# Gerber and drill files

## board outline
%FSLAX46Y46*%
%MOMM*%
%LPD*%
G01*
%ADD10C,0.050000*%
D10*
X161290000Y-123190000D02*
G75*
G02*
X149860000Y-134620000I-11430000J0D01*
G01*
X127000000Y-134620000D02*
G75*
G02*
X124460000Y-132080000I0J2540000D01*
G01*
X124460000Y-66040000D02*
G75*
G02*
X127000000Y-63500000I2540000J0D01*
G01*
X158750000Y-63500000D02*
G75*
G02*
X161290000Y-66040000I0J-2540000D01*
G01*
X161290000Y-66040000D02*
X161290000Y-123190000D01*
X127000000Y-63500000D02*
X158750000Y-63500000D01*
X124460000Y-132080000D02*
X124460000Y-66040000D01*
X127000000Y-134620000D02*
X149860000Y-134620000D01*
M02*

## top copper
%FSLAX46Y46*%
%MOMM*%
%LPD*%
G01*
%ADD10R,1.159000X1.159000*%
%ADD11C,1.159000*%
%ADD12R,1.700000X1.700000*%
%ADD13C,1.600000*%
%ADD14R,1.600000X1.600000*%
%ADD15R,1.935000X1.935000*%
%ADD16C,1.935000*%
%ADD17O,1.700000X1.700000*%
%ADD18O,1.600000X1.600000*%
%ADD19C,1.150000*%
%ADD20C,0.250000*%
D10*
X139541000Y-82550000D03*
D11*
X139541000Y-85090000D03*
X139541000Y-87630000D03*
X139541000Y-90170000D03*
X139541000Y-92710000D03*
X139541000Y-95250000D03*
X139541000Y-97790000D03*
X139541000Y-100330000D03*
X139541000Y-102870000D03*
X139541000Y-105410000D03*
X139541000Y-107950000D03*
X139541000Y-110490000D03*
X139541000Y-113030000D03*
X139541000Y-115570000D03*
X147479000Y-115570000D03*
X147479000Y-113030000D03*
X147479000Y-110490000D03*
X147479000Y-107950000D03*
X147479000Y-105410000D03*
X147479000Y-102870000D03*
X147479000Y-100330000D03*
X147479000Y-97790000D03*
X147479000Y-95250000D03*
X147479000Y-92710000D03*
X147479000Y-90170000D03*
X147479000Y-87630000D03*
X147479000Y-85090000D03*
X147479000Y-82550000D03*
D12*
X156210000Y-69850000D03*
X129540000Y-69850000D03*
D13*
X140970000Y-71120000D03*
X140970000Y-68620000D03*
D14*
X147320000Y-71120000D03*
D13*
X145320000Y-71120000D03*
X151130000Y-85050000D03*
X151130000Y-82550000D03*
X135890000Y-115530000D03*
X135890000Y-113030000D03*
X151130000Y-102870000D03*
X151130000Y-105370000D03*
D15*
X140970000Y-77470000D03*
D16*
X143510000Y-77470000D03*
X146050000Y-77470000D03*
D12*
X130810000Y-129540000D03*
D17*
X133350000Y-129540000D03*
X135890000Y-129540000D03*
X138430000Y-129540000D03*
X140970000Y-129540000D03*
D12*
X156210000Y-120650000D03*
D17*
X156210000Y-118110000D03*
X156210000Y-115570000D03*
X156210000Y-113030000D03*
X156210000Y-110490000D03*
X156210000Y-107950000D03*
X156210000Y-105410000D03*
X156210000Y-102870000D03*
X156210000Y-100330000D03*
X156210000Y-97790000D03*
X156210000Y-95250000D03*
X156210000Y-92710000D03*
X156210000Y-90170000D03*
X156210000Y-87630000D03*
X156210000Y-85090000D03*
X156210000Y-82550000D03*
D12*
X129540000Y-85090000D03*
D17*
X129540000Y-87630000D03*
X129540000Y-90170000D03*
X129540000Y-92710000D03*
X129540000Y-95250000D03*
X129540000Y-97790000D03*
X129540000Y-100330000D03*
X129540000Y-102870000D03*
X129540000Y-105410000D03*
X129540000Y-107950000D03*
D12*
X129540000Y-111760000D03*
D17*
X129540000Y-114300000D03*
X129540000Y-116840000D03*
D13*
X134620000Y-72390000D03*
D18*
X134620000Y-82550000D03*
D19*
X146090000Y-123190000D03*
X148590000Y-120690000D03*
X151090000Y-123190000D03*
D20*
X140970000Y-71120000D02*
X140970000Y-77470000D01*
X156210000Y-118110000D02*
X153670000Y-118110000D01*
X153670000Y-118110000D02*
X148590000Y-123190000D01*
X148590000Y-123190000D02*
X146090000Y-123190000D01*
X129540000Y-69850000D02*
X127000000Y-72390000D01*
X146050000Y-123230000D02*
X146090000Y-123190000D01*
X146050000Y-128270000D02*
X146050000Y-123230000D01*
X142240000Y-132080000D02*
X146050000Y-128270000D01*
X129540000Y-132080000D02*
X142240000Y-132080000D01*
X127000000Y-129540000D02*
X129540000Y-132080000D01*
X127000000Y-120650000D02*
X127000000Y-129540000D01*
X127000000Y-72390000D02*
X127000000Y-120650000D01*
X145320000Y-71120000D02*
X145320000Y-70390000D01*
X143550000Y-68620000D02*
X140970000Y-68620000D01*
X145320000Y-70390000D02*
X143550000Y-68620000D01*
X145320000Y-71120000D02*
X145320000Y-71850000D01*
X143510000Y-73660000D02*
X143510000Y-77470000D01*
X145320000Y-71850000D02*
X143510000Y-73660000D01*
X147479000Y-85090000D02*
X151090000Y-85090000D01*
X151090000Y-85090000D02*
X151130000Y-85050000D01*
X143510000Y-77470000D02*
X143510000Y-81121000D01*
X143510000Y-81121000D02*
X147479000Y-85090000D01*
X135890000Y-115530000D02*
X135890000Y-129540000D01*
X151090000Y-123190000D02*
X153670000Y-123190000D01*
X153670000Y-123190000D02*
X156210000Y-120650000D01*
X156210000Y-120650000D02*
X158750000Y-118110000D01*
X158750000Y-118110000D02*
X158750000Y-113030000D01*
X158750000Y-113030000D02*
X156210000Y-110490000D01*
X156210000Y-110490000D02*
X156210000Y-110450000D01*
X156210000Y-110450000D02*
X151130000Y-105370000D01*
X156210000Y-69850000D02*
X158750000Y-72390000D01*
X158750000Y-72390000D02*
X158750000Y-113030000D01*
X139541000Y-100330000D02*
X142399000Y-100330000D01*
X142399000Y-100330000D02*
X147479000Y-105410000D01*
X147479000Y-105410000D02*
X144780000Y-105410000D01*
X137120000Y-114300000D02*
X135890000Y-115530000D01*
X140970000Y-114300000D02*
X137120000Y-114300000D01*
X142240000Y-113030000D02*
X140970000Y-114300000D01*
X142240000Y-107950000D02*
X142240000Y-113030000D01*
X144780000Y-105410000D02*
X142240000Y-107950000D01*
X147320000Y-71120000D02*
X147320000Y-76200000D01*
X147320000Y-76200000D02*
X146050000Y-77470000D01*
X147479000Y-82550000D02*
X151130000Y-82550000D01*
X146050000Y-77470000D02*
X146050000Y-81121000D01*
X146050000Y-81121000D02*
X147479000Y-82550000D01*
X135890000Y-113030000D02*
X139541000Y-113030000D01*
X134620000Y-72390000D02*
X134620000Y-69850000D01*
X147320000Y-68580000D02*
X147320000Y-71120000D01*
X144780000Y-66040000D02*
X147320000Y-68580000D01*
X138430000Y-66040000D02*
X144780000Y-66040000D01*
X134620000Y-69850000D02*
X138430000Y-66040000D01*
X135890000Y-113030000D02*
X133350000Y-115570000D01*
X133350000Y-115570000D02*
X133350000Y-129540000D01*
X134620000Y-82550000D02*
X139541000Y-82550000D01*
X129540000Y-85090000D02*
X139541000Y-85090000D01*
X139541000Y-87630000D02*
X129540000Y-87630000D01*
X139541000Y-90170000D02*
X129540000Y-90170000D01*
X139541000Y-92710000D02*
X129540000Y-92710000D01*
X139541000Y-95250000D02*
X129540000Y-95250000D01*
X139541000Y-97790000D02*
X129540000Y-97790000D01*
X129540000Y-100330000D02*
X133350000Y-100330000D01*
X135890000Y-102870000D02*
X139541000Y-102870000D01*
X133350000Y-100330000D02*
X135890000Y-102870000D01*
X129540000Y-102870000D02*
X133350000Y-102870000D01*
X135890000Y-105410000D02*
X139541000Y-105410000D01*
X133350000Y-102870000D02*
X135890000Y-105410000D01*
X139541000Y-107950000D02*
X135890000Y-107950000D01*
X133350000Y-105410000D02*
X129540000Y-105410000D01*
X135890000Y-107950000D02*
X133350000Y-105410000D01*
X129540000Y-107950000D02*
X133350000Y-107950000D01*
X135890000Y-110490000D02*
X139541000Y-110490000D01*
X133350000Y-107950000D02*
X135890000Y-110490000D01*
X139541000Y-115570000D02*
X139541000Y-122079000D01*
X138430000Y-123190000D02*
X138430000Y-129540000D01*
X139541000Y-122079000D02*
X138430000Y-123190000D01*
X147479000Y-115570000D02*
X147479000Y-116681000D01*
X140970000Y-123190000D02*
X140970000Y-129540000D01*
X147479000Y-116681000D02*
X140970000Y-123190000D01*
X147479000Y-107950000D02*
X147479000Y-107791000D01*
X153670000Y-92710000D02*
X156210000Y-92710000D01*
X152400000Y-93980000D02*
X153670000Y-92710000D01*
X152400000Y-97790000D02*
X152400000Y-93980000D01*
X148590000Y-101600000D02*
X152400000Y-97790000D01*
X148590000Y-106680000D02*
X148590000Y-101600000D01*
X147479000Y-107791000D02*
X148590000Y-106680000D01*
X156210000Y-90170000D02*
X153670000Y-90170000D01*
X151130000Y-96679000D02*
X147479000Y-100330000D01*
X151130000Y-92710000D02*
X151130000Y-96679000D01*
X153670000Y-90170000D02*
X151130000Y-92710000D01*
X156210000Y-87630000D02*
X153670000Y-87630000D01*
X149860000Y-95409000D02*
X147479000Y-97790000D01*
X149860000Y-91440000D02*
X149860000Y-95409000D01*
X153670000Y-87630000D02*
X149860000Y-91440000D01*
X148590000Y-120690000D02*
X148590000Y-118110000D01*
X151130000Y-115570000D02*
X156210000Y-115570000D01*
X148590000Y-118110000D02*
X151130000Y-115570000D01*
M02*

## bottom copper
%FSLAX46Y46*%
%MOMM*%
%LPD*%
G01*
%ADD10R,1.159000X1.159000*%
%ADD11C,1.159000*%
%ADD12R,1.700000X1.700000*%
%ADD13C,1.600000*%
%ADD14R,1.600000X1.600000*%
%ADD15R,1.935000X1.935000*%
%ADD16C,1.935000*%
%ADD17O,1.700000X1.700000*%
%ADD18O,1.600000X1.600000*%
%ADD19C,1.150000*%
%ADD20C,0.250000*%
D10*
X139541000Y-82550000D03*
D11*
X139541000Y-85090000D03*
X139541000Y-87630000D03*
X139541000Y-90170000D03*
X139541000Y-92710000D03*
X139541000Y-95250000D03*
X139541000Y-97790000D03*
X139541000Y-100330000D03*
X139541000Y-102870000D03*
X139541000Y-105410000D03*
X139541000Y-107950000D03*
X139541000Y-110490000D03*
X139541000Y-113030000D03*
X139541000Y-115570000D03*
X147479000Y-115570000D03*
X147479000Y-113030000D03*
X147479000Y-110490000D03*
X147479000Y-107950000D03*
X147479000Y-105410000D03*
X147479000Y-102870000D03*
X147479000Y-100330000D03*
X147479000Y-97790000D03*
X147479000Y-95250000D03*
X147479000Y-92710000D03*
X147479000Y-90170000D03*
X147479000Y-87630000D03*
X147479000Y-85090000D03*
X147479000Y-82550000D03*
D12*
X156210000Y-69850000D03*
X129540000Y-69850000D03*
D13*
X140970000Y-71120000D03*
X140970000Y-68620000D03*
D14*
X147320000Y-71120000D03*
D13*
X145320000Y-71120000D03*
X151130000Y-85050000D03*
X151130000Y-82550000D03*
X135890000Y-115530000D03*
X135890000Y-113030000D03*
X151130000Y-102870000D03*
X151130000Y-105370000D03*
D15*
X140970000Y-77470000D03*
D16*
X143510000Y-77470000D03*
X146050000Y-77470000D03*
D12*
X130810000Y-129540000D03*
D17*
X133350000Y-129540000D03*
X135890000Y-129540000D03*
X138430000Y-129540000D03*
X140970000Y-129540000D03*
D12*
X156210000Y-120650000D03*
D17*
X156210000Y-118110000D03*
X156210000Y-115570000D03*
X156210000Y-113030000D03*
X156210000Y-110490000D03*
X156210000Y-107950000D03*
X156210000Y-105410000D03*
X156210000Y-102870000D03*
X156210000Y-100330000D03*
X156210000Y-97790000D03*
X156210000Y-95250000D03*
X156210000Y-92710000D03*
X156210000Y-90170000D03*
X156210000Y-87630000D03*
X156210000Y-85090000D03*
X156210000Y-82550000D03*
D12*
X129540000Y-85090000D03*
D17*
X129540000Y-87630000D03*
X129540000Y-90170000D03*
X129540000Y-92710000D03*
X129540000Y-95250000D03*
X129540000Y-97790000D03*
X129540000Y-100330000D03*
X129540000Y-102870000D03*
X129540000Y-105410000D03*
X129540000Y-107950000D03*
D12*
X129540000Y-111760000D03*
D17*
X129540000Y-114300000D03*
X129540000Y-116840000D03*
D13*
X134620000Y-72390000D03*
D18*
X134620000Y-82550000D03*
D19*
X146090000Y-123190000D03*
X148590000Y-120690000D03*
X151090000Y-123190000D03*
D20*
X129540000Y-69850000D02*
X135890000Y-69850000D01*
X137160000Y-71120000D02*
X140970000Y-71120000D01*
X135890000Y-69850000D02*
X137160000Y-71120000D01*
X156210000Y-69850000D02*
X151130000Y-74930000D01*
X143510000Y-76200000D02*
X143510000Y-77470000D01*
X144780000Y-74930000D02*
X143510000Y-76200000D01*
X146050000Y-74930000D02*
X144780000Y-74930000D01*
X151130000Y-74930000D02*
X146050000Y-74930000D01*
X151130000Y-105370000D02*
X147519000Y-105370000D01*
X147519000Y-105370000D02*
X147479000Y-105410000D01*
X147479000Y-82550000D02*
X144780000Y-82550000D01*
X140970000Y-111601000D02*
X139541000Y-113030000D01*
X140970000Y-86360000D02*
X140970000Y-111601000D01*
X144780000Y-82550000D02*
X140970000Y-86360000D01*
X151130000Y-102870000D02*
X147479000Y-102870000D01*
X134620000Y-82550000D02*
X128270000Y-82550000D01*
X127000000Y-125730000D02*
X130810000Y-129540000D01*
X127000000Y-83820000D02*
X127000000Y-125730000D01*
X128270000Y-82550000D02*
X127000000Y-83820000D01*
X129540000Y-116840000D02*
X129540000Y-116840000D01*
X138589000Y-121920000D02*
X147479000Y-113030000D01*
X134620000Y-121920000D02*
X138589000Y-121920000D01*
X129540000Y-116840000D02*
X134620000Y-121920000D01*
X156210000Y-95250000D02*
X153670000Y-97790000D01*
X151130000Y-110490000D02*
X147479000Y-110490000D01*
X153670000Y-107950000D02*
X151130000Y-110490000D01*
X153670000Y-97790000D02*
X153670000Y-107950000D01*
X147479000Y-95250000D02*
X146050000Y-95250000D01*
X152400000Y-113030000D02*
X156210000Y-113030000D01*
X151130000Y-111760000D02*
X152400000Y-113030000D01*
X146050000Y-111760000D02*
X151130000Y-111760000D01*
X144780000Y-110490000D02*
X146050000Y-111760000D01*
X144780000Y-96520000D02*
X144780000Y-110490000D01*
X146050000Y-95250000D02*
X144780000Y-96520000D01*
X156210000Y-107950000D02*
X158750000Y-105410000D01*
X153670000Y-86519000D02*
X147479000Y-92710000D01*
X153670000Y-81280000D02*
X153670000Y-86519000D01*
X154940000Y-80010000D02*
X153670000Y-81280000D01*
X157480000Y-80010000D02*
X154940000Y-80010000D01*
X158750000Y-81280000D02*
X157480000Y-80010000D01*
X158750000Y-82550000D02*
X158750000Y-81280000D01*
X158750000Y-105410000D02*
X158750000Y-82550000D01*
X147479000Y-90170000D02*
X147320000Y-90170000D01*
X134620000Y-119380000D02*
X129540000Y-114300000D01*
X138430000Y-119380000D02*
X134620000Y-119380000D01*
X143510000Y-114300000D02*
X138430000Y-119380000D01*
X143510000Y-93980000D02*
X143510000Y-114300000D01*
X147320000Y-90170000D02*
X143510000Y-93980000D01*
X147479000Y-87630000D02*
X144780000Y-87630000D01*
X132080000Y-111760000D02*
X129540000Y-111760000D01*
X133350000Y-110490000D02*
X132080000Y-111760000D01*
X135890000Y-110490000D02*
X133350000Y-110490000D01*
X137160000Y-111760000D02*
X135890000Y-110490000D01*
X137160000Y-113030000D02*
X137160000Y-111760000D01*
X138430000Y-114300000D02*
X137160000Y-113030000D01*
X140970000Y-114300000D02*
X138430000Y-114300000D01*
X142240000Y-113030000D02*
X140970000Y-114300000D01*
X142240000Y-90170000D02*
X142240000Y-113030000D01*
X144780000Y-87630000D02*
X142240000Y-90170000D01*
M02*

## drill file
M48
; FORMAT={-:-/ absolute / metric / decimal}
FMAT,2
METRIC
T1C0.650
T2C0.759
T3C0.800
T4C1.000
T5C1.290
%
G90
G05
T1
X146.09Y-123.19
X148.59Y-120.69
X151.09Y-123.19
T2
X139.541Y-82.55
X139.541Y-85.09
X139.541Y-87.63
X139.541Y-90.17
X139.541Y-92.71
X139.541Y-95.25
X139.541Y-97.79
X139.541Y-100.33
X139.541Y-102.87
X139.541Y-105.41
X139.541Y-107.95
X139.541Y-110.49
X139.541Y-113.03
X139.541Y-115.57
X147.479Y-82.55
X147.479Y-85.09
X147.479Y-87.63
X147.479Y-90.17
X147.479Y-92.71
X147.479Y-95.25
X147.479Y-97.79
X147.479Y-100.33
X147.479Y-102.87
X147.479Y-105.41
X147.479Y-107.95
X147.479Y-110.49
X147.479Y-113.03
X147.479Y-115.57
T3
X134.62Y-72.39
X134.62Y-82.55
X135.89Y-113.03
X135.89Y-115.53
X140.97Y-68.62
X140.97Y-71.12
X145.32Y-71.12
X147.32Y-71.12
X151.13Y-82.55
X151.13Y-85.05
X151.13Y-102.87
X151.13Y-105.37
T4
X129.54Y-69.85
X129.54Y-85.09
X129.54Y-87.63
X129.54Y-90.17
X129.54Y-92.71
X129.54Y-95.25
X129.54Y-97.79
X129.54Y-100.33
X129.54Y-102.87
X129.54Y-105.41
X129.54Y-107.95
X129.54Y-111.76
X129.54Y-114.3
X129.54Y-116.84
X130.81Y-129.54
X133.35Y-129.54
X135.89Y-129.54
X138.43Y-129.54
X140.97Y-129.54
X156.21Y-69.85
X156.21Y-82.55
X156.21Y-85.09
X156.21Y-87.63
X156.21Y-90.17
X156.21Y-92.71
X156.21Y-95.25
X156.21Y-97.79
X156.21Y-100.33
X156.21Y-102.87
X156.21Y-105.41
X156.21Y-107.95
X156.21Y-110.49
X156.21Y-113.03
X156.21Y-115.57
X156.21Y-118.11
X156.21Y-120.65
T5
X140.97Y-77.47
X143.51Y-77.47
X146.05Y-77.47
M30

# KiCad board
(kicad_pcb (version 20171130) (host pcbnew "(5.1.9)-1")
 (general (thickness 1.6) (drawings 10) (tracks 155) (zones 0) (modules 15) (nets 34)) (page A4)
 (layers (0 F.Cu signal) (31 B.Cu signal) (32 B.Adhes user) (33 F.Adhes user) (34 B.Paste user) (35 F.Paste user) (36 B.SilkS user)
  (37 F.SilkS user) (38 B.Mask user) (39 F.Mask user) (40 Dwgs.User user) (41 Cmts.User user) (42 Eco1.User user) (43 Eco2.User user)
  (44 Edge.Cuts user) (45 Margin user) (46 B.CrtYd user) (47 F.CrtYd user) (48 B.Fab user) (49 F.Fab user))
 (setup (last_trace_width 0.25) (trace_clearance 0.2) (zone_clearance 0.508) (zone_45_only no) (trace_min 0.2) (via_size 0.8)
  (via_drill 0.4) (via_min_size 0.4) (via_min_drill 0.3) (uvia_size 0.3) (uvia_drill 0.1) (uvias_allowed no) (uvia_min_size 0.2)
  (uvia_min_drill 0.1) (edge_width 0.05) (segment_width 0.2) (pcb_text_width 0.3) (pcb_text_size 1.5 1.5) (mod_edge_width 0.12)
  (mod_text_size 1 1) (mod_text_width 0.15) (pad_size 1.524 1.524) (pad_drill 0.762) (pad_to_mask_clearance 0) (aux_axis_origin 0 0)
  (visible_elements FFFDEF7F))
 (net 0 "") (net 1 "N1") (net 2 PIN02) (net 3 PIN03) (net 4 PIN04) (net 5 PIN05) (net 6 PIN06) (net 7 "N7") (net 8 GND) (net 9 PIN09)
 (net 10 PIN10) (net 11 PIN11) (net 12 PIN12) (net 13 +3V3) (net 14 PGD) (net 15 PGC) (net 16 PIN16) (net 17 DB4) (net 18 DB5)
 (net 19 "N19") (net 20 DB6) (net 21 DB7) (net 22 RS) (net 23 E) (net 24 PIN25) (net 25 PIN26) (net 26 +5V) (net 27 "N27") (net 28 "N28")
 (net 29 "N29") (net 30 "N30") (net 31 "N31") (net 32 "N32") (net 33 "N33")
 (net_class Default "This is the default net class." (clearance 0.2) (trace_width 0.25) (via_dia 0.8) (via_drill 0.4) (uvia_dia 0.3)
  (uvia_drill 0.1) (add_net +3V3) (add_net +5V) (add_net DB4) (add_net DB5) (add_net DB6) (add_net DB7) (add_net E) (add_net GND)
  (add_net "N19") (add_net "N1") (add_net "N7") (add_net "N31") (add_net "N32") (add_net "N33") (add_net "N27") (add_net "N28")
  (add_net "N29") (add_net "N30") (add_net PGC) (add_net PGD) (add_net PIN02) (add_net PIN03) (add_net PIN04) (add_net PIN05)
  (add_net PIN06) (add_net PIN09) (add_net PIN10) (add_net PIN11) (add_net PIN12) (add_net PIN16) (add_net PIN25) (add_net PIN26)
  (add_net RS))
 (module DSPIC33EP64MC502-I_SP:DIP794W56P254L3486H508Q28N (layer F.Cu) (at 143.51 99.06)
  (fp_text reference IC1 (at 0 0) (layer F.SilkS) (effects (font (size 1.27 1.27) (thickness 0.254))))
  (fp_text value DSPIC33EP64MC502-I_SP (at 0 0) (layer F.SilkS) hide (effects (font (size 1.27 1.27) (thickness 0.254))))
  (pad 1 thru_hole rect (at -3.969 -16.51 90) (size 1.159 1.159) (drill 0.759) (layers *.Cu *.Mask F.SilkS) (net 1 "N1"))
  (pad 2 thru_hole circle (at -3.969 -13.97 90) (size 1.159 1.159) (drill 0.759) (layers *.Cu *.Mask F.SilkS) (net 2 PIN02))
  (pad 3 thru_hole circle (at -3.969 -11.43 90) (size 1.159 1.159) (drill 0.759) (layers *.Cu *.Mask F.SilkS) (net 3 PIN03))
  (pad 4 thru_hole circle (at -3.969 -8.89 90) (size 1.159 1.159) (drill 0.759) (layers *.Cu *.Mask F.SilkS) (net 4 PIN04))
  (pad 5 thru_hole circle (at -3.969 -6.35 90) (size 1.159 1.159) (drill 0.759) (layers *.Cu *.Mask F.SilkS) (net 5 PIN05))
  (pad 6 thru_hole circle (at -3.969 -3.81 90) (size 1.159 1.159) (drill 0.759) (layers *.Cu *.Mask F.SilkS) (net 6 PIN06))
  (pad 7 thru_hole circle (at -3.969 -1.27 90) (size 1.159 1.159) (drill 0.759) (layers *.Cu *.Mask F.SilkS) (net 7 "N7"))
  (pad 8 thru_hole circle (at -3.969 1.27 90) (size 1.159 1.159) (drill 0.759) (layers *.Cu *.Mask F.SilkS) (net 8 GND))
  (pad 9 thru_hole circle (at -3.969 3.81 90) (size 1.159 1.159) (drill 0.759) (layers *.Cu *.Mask F.SilkS) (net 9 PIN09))
  (pad 10 thru_hole circle (at -3.969 6.35 90) (size 1.159 1.159) (drill 0.759) (layers *.Cu *.Mask F.SilkS) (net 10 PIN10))
  (pad 11 thru_hole circle (at -3.969 8.89 90) (size 1.159 1.159) (drill 0.759) (layers *.Cu *.Mask F.SilkS) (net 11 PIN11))
  (pad 12 thru_hole circle (at -3.969 11.43 90) (size 1.159 1.159) (drill 0.759) (layers *.Cu *.Mask F.SilkS) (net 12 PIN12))
  (pad 13 thru_hole circle (at -3.969 13.97 90) (size 1.159 1.159) (drill 0.759) (layers *.Cu *.Mask F.SilkS) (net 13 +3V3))
  (pad 14 thru_hole circle (at -3.969 16.51 90) (size 1.159 1.159) (drill 0.759) (layers *.Cu *.Mask F.SilkS) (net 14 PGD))
  (pad 15 thru_hole circle (at 3.969 16.51 90) (size 1.159 1.159) (drill 0.759) (layers *.Cu *.Mask F.SilkS) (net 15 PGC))
  (pad 16 thru_hole circle (at 3.969 13.97 90) (size 1.159 1.159) (drill 0.759) (layers *.Cu *.Mask F.SilkS) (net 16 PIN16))
  (pad 17 thru_hole circle (at 3.969 11.43 90) (size 1.159 1.159) (drill 0.759) (layers *.Cu *.Mask F.SilkS) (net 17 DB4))
  (pad 18 thru_hole circle (at 3.969 8.89 90) (size 1.159 1.159) (drill 0.759) (layers *.Cu *.Mask F.SilkS) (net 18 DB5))
  (pad 19 thru_hole circle (at 3.969 6.35 90) (size 1.159 1.159) (drill 0.759) (layers *.Cu *.Mask F.SilkS) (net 8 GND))
  (pad 20 thru_hole circle (at 3.969 3.81 90) (size 1.159 1.159) (drill 0.759) (layers *.Cu *.Mask F.SilkS) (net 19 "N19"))
  (pad 21 thru_hole circle (at 3.969 1.27 90) (size 1.159 1.159) (drill 0.759) (layers *.Cu *.Mask F.SilkS) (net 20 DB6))
  (pad 22 thru_hole circle (at 3.969 -1.27 90) (size 1.159 1.159) (drill 0.759) (layers *.Cu *.Mask F.SilkS) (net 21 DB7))
  (pad 23 thru_hole circle (at 3.969 -3.81 90) (size 1.159 1.159) (drill 0.759) (layers *.Cu *.Mask F.SilkS) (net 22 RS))
  (pad 24 thru_hole circle (at 3.969 -6.35 90) (size 1.159 1.159) (drill 0.759) (layers *.Cu *.Mask F.SilkS) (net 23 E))
  (pad 25 thru_hole circle (at 3.969 -8.89 90) (size 1.159 1.159) (drill 0.759) (layers *.Cu *.Mask F.SilkS) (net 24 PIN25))
  (pad 26 thru_hole circle (at 3.969 -11.43 90) (size 1.159 1.159) (drill 0.759) (layers *.Cu *.Mask F.SilkS) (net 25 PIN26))
  (pad 27 thru_hole circle (at 3.969 -13.97 90) (size 1.159 1.159) (drill 0.759) (layers *.Cu *.Mask F.SilkS) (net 8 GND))
  (pad 28 thru_hole circle (at 3.969 -16.51 90) (size 1.159 1.159) (drill 0.759) (layers *.Cu *.Mask F.SilkS) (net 13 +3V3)))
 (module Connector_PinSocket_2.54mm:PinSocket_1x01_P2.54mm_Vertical (layer F.Cu) (at 156.21 69.85)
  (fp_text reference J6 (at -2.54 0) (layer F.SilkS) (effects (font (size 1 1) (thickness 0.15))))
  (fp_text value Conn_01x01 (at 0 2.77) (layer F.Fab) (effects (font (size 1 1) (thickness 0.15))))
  (pad 1 thru_hole rect (at 0 0) (size 1.7 1.7) (drill 1) (layers *.Cu *.Mask) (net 8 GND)))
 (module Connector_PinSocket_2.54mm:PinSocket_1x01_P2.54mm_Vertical (layer F.Cu) (at 129.54 69.85)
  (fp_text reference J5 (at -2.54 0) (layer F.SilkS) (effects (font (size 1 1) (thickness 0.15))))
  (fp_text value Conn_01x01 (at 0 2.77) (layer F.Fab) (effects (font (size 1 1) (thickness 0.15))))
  (pad 1 thru_hole rect (at 0 0) (size 1.7 1.7) (drill 1) (layers *.Cu *.Mask) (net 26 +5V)))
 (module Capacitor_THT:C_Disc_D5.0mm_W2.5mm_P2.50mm (layer F.Cu) (at 140.97 71.12 90)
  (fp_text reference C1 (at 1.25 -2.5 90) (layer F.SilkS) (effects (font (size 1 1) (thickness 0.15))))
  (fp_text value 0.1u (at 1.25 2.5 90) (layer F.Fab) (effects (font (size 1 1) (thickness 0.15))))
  (pad 1 thru_hole circle (at 0 0 90) (size 1.6 1.6) (drill 0.8) (layers *.Cu *.Mask) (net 26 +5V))
  (pad 2 thru_hole circle (at 2.5 0 90) (size 1.6 1.6) (drill 0.8) (layers *.Cu *.Mask) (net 8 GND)))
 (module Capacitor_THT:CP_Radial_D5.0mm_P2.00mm (layer F.Cu) (at 147.32 71.12 180)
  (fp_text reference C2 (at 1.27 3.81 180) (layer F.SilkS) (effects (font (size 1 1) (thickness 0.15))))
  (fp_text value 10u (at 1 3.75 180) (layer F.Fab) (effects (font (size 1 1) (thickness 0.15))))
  (pad 1 thru_hole rect (at 0 0 180) (size 1.6 1.6) (drill 0.8) (layers *.Cu *.Mask) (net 13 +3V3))
  (pad 2 thru_hole circle (at 2 0 180) (size 1.6 1.6) (drill 0.8) (layers *.Cu *.Mask) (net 8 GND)))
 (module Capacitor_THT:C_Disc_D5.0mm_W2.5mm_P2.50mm (layer F.Cu) (at 151.13 82.55 270)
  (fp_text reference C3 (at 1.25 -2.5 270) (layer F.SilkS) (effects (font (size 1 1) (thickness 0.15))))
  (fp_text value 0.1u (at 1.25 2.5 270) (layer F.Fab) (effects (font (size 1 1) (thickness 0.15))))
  (pad 2 thru_hole circle (at 2.5 0 270) (size 1.6 1.6) (drill 0.8) (layers *.Cu *.Mask) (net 8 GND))
  (pad 1 thru_hole circle (at 0 0 270) (size 1.6 1.6) (drill 0.8) (layers *.Cu *.Mask) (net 13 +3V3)))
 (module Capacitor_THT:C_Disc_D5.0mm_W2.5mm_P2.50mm (layer F.Cu) (at 135.89 113.03 270)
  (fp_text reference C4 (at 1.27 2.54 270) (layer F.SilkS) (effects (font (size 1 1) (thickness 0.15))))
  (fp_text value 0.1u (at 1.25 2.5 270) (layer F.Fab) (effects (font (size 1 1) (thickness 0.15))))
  (pad 2 thru_hole circle (at 2.5 0 270) (size 1.6 1.6) (drill 0.8) (layers *.Cu *.Mask) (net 8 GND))
  (pad 1 thru_hole circle (at 0 0 270) (size 1.6 1.6) (drill 0.8) (layers *.Cu *.Mask) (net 13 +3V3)))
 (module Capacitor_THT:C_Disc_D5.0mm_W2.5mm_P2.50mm (layer F.Cu) (at 151.13 102.87 270)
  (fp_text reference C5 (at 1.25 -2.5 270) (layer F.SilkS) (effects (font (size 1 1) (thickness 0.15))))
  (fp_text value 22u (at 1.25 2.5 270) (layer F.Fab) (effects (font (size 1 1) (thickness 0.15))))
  (pad 1 thru_hole circle (at 0 0 270) (size 1.6 1.6) (drill 0.8) (layers *.Cu *.Mask) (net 19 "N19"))
  (pad 2 thru_hole circle (at 2.5 0 270) (size 1.6 1.6) (drill 0.8) (layers *.Cu *.Mask) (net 8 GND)))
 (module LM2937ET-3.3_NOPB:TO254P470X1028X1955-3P (layer F.Cu) (at 140.97 77.47)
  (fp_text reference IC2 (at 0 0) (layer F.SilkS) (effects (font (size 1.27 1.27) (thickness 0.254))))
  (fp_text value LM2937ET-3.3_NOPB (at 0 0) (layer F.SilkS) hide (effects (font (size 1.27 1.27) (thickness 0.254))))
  (pad 1 thru_hole rect (at 0 0 90) (size 1.935 1.935) (drill 1.29) (layers *.Cu *.Mask F.SilkS) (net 26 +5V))
  (pad 2 thru_hole circle (at 2.54 0 90) (size 1.935 1.935) (drill 1.29) (layers *.Cu *.Mask F.SilkS) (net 8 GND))
  (pad 3 thru_hole circle (at 5.08 0 90) (size 1.935 1.935) (drill 1.29) (layers *.Cu *.Mask F.SilkS) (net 13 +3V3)))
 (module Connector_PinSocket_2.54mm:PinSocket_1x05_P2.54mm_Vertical (layer F.Cu) (at 130.81 129.54 90)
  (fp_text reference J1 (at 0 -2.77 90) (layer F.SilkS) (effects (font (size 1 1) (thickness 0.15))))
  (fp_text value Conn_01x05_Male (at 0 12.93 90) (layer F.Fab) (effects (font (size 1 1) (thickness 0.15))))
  (pad 1 thru_hole rect (at 0 0 90) (size 1.7 1.7) (drill 1) (layers *.Cu *.Mask) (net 1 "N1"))
  (pad 2 thru_hole oval (at 0 2.54 90) (size 1.7 1.7) (drill 1) (layers *.Cu *.Mask) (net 13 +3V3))
  (pad 3 thru_hole oval (at 0 5.08 90) (size 1.7 1.7) (drill 1) (layers *.Cu *.Mask) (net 8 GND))
  (pad 4 thru_hole oval (at 0 7.62 90) (size 1.7 1.7) (drill 1) (layers *.Cu *.Mask) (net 14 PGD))
  (pad 5 thru_hole oval (at 0 10.16 90) (size 1.7 1.7) (drill 1) (layers *.Cu *.Mask) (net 15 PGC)))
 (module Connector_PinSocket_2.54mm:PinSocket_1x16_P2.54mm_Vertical (layer F.Cu) (at 156.21 120.65 180)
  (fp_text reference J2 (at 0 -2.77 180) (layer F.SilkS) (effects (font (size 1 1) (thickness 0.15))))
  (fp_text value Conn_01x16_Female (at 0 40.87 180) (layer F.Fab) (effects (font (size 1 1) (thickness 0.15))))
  (pad 1 thru_hole rect (at 0 0 180) (size 1.7 1.7) (drill 1) (layers *.Cu *.Mask) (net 8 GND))
  (pad 2 thru_hole oval (at 0 2.54 180) (size 1.7 1.7) (drill 1) (layers *.Cu *.Mask) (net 26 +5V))
  (pad 3 thru_hole oval (at 0 5.08 180) (size 1.7 1.7) (drill 1) (layers *.Cu *.Mask) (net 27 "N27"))
  (pad 4 thru_hole oval (at 0 7.62 180) (size 1.7 1.7) (drill 1) (layers *.Cu *.Mask) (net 22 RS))
  (pad 5 thru_hole oval (at 0 10.16 180) (size 1.7 1.7) (drill 1) (layers *.Cu *.Mask) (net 8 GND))
  (pad 6 thru_hole oval (at 0 12.7 180) (size 1.7 1.7) (drill 1) (layers *.Cu *.Mask) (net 23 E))
  (pad 7 thru_hole oval (at 0 15.24 180) (size 1.7 1.7) (drill 1) (layers *.Cu *.Mask) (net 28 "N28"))
  (pad 8 thru_hole oval (at 0 17.78 180) (size 1.7 1.7) (drill 1) (layers *.Cu *.Mask) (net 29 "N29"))
  (pad 9 thru_hole oval (at 0 20.32 180) (size 1.7 1.7) (drill 1) (layers *.Cu *.Mask) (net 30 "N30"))
  (pad 10 thru_hole oval (at 0 22.86 180) (size 1.7 1.7) (drill 1) (layers *.Cu *.Mask) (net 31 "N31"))
  (pad 11 thru_hole oval (at 0 25.4 180) (size 1.7 1.7) (drill 1) (layers *.Cu *.Mask) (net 17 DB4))
  (pad 12 thru_hole oval (at 0 27.94 180) (size 1.7 1.7) (drill 1) (layers *.Cu *.Mask) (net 18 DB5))
  (pad 13 thru_hole oval (at 0 30.48 180) (size 1.7 1.7) (drill 1) (layers *.Cu *.Mask) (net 20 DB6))
  (pad 14 thru_hole oval (at 0 33.02 180) (size 1.7 1.7) (drill 1) (layers *.Cu *.Mask) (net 21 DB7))
  (pad 15 thru_hole oval (at 0 35.56 180) (size 1.7 1.7) (drill 1) (layers *.Cu *.Mask) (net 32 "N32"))
  (pad 16 thru_hole oval (at 0 38.1 180) (size 1.7 1.7) (drill 1) (layers *.Cu *.Mask) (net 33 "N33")))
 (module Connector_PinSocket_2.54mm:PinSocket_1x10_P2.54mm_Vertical (layer F.Cu) (at 129.54 85.09)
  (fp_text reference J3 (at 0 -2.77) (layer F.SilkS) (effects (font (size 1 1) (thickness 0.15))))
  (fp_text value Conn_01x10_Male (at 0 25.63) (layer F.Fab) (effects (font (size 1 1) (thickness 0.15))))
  (pad 1 thru_hole rect (at 0 0) (size 1.7 1.7) (drill 1) (layers *.Cu *.Mask) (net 2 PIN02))
  (pad 2 thru_hole oval (at 0 2.54) (size 1.7 1.7) (drill 1) (layers *.Cu *.Mask) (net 3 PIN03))
  (pad 3 thru_hole oval (at 0 5.08) (size 1.7 1.7) (drill 1) (layers *.Cu *.Mask) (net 4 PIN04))
  (pad 4 thru_hole oval (at 0 7.62) (size 1.7 1.7) (drill 1) (layers *.Cu *.Mask) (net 5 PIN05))
  (pad 5 thru_hole oval (at 0 10.16) (size 1.7 1.7) (drill 1) (layers *.Cu *.Mask) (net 6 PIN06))
  (pad 6 thru_hole oval (at 0 12.7) (size 1.7 1.7) (drill 1) (layers *.Cu *.Mask) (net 7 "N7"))
  (pad 7 thru_hole oval (at 0 15.24) (size 1.7 1.7) (drill 1) (layers *.Cu *.Mask) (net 9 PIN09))
  (pad 8 thru_hole oval (at 0 17.78) (size 1.7 1.7) (drill 1) (layers *.Cu *.Mask) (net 10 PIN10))
  (pad 9 thru_hole oval (at 0 20.32) (size 1.7 1.7) (drill 1) (layers *.Cu *.Mask) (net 11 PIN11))
  (pad 10 thru_hole oval (at 0 22.86) (size 1.7 1.7) (drill 1) (layers *.Cu *.Mask) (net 12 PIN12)))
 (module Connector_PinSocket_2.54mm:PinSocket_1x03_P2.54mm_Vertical (layer F.Cu) (at 129.54 111.76)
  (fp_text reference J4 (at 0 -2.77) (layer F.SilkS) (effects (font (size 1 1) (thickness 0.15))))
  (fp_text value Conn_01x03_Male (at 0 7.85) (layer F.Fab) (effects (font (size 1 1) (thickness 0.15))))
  (pad 1 thru_hole rect (at 0 0) (size 1.7 1.7) (drill 1) (layers *.Cu *.Mask) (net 25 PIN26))
  (pad 2 thru_hole oval (at 0 2.54) (size 1.7 1.7) (drill 1) (layers *.Cu *.Mask) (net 24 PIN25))
  (pad 3 thru_hole oval (at 0 5.08) (size 1.7 1.7) (drill 1) (layers *.Cu *.Mask) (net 16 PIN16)))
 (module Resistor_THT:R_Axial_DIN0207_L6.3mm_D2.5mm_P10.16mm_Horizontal (layer F.Cu) (at 134.62 72.39 270)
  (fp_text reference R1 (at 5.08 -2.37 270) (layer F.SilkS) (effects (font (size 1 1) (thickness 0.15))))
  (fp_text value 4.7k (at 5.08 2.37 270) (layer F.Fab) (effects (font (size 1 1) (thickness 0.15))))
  (pad 1 thru_hole circle (at 0 0 270) (size 1.6 1.6) (drill 0.8) (layers *.Cu *.Mask) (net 13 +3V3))
  (pad 2 thru_hole oval (at 10.16 0 270) (size 1.6 1.6) (drill 0.8) (layers *.Cu *.Mask) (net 1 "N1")))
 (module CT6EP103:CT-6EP (layer F.Cu) (at 148.59 123.19)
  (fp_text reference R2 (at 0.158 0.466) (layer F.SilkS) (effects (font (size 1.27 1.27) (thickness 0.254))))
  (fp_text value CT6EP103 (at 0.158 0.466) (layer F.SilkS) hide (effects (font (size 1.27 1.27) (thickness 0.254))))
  (pad 1 thru_hole circle (at -2.5 0 90) (size 1.15 1.15) (drill 0.65) (layers *.Cu *.Mask F.SilkS) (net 26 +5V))
  (pad 2 thru_hole circle (at 0 -2.5 90) (size 1.15 1.15) (drill 0.65) (layers *.Cu *.Mask F.SilkS) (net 27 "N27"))
  (pad 3 thru_hole circle (at 2.5 0 90) (size 1.15 1.15) (drill 0.65) (layers *.Cu *.Mask F.SilkS) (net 8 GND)))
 (gr_arc (start 149.86 123.19) (end 161.29 123.19) (angle 90) (layer Edge.Cuts) (width 0.05))
 (gr_arc (start 127 132.08) (end 127 134.62) (angle 90) (layer Edge.Cuts) (width 0.05))
 (gr_arc (start 127 66.04) (end 124.46 66.04) (angle 90) (layer Edge.Cuts) (width 0.05))
 (gr_arc (start 158.75 66.04) (end 158.75 63.5) (angle 90) (layer Edge.Cuts) (width 0.05))
 (gr_line (start 161.29 66.04) (end 161.29 123.19) (angle 90) (layer Edge.Cuts) (width 0.05))
 (gr_line (start 127 63.5) (end 158.75 63.5) (angle 90) (layer Edge.Cuts) (width 0.05))
 (gr_line (start 124.46 132.08) (end 124.46 66.04) (angle 90) (layer Edge.Cuts) (width 0.05))
 (gr_line (start 127 134.62) (end 149.86 134.62) (angle 90) (layer Edge.Cuts) (width 0.05))
 (segment (start 140.97 71.12) (end 140.97 77.47) (width 0.25) (layer F.Cu) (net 26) (status C00000))
 (segment (start 156.21 118.11) (end 153.67 118.11) (width 0.25) (layer F.Cu) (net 26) (status 400000))
 (segment (start 153.67 118.11) (end 148.59 123.19) (width 0.25) (layer F.Cu) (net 26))
 (segment (start 148.59 123.19) (end 146.09 123.19) (width 0.25) (layer F.Cu) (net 26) (status 800000))
 (segment (start 129.54 69.85) (end 135.89 69.85) (width 0.25) (layer B.Cu) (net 26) (status 400000))
 (segment (start 137.16 71.12) (end 140.97 71.12) (width 0.25) (layer B.Cu) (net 26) (status 800000))
 (segment (start 135.89 69.85) (end 137.16 71.12) (width 0.25) (layer B.Cu) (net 26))
 (segment (start 129.54 69.85) (end 127 72.39) (width 0.25) (layer F.Cu) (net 26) (status 400000))
 (segment (start 146.05 123.23) (end 146.09 123.19) (width 0.25) (layer F.Cu) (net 26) (status C00000))
 (segment (start 146.05 128.27) (end 146.05 123.23) (width 0.25) (layer F.Cu) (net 26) (status 800000))
 (segment (start 142.24 132.08) (end 146.05 128.27) (width 0.25) (layer F.Cu) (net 26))
 (segment (start 129.54 132.08) (end 142.24 132.08) (width 0.25) (layer F.Cu) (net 26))
 (segment (start 127 129.54) (end 129.54 132.08) (width 0.25) (layer F.Cu) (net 26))
 (segment (start 127 120.65) (end 127 129.54) (width 0.25) (layer F.Cu) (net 26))
 (segment (start 127 72.39) (end 127 120.65) (width 0.25) (layer F.Cu) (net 26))
 (segment (start 145.32 71.12) (end 145.32 70.39) (width 0.25) (layer F.Cu) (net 8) (status C00000))
 (segment (start 143.55 68.62) (end 140.97 68.62) (width 0.25) (layer F.Cu) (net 8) (status 800000))
 (segment (start 145.32 70.39) (end 143.55 68.62) (width 0.25) (layer F.Cu) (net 8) (status 400000))
 (segment (start 145.32 71.12) (end 145.32 71.85) (width 0.25) (layer F.Cu) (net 8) (status C00000))
 (segment (start 143.51 73.66) (end 143.51 77.47) (width 0.25) (layer F.Cu) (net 8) (status 800000))
 (segment (start 145.32 71.85) (end 143.51 73.66) (width 0.25) (layer F.Cu) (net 8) (status 400000))
 (segment (start 147.479 85.09) (end 151.09 85.09) (width 0.25) (layer F.Cu) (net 8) (status C00000))
 (segment (start 151.09 85.09) (end 151.13 85.05) (width 0.25) (layer F.Cu) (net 8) (status C00000))
 (segment (start 143.51 77.47) (end 143.51 81.121) (width 0.25) (layer F.Cu) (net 8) (status 400000))
 (segment (start 143.51 81.121) (end 147.479 85.09) (width 0.25) (layer F.Cu) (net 8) (status 800000))
 (segment (start 135.89 115.53) (end 135.89 129.54) (width 0.25) (layer F.Cu) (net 8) (status C00000))
 (segment (start 151.09 123.19) (end 153.67 123.19) (width 0.25) (layer F.Cu) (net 8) (status 400000))
 (segment (start 153.67 123.19) (end 156.21 120.65) (width 0.25) (layer F.Cu) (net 8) (status 800000))
 (segment (start 156.21 69.85) (end 151.13 74.93) (width 0.25) (layer B.Cu) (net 8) (status 400000))
 (segment (start 143.51 76.2) (end 143.51 77.47) (width 0.25) (layer B.Cu) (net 8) (status 800000))
 (segment (start 144.78 74.93) (end 143.51 76.2) (width 0.25) (layer B.Cu) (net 8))
 (segment (start 146.05 74.93) (end 144.78 74.93) (width 0.25) (layer B.Cu) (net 8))
 (segment (start 151.13 74.93) (end 146.05 74.93) (width 0.25) (layer B.Cu) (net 8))
 (segment (start 156.21 120.65) (end 158.75 118.11) (width 0.25) (layer F.Cu) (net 8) (status 400000))
 (segment (start 158.75 118.11) (end 158.75 113.03) (width 0.25) (layer F.Cu) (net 8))
 (segment (start 158.75 113.03) (end 156.21 110.49) (width 0.25) (layer F.Cu) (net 8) (status 800000))
 (segment (start 156.21 110.49) (end 156.21 110.45) (width 0.25) (layer F.Cu) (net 8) (status C00000))
 (segment (start 156.21 110.45) (end 151.13 105.37) (width 0.25) (layer F.Cu) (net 8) (status C00000))
 (segment (start 156.21 69.85) (end 158.75 72.39) (width 0.25) (layer F.Cu) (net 8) (status 400000))
 (segment (start 158.75 72.39) (end 158.75 113.03) (width 0.25) (layer F.Cu) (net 8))
 (segment (start 151.13 105.37) (end 147.519 105.37) (width 0.25) (layer B.Cu) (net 8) (status C00000))
 (segment (start 147.519 105.37) (end 147.479 105.41) (width 0.25) (layer B.Cu) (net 8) (status C00000))
 (segment (start 139.541 100.33) (end 142.399 100.33) (width 0.25) (layer F.Cu) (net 8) (status 400000))
 (segment (start 142.399 100.33) (end 147.479 105.41) (width 0.25) (layer F.Cu) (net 8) (status 800000))
 (segment (start 147.479 105.41) (end 144.78 105.41) (width 0.25) (layer F.Cu) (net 8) (status 400000))
 (segment (start 137.12 114.3) (end 135.89 115.53) (width 0.25) (layer F.Cu) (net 8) (status 800000))
 (segment (start 140.97 114.3) (end 137.12 114.3) (width 0.25) (layer F.Cu) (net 8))
 (segment (start 142.24 113.03) (end 140.97 114.3) (width 0.25) (layer F.Cu) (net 8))
 (segment (start 142.24 107.95) (end 142.24 113.03) (width 0.25) (layer F.Cu) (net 8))
 (segment (start 144.78 105.41) (end 142.24 107.95) (width 0.25) (layer F.Cu) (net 8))
 (segment (start 147.32 71.12) (end 147.32 76.2) (width 0.25) (layer F.Cu) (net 13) (status 400000))
 (segment (start 147.32 76.2) (end 146.05 77.47) (width 0.25) (layer F.Cu) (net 13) (status 800000))
 (segment (start 147.479 82.55) (end 151.13 82.55) (width 0.25) (layer F.Cu) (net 13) (status C00000))
 (segment (start 146.05 77.47) (end 146.05 81.121) (width 0.25) (layer F.Cu) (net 13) (status 400000))
 (segment (start 146.05 81.121) (end 147.479 82.55) (width 0.25) (layer F.Cu) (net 13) (status 800000))
 (segment (start 135.89 113.03) (end 139.541 113.03) (width 0.25) (layer F.Cu) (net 13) (status C00000))
 (segment (start 134.62 72.39) (end 134.62 69.85) (width 0.25) (layer F.Cu) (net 13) (status 400000))
 (segment (start 147.32 68.58) (end 147.32 71.12) (width 0.25) (layer F.Cu) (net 13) (status 800000))
 (segment (start 144.78 66.04) (end 147.32 68.58) (width 0.25) (layer F.Cu) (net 13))
 (segment (start 138.43 66.04) (end 144.78 66.04) (width 0.25) (layer F.Cu) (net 13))
 (segment (start 134.62 69.85) (end 138.43 66.04) (width 0.25) (layer F.Cu) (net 13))
 (segment (start 135.89 113.03) (end 133.35 115.57) (width 0.25) (layer F.Cu) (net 13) (status 400000))
 (segment (start 133.35 115.57) (end 133.35 129.54) (width 0.25) (layer F.Cu) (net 13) (status 800000))
 (segment (start 147.479 82.55) (end 144.78 82.55) (width 0.25) (layer B.Cu) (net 13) (status 400000))
 (segment (start 140.97 111.601) (end 139.541 113.03) (width 0.25) (layer B.Cu) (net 13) (status 800000))
 (segment (start 140.97 86.36) (end 140.97 111.601) (width 0.25) (layer B.Cu) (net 13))
 (segment (start 144.78 82.55) (end 140.97 86.36) (width 0.25) (layer B.Cu) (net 13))
 (segment (start 151.13 102.87) (end 147.479 102.87) (width 0.25) (layer B.Cu) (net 19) (status C00000))
 (segment (start 134.62 82.55) (end 139.541 82.55) (width 0.25) (layer F.Cu) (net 1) (status C00000))
 (segment (start 134.62 82.55) (end 128.27 82.55) (width 0.25) (layer B.Cu) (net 1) (status 400000))
 (segment (start 127 125.73) (end 130.81 129.54) (width 0.25) (layer B.Cu) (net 1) (status 800000))
 (segment (start 127 83.82) (end 127 125.73) (width 0.25) (layer B.Cu) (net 1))
 (segment (start 128.27 82.55) (end 127 83.82) (width 0.25) (layer B.Cu) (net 1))
 (segment (start 129.54 85.09) (end 139.541 85.09) (width 0.25) (layer F.Cu) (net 2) (status C00000))
 (segment (start 139.541 87.63) (end 129.54 87.63) (width 0.25) (layer F.Cu) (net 3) (status C00000))
 (segment (start 139.541 90.17) (end 129.54 90.17) (width 0.25) (layer F.Cu) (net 4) (status C00000))
 (segment (start 139.541 92.71) (end 129.54 92.71) (width 0.25) (layer F.Cu) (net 5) (status C00000))
 (segment (start 139.541 95.25) (end 129.54 95.25) (width 0.25) (layer F.Cu) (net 6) (status C00000))
 (segment (start 139.541 97.79) (end 129.54 97.79) (width 0.25) (layer F.Cu) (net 7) (status C00000))
 (segment (start 129.54 100.33) (end 133.35 100.33) (width 0.25) (layer F.Cu) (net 9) (status 400000))
 (segment (start 135.89 102.87) (end 139.541 102.87) (width 0.25) (layer F.Cu) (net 9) (status 800000))
 (segment (start 133.35 100.33) (end 135.89 102.87) (width 0.25) (layer F.Cu) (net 9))
 (segment (start 129.54 102.87) (end 133.35 102.87) (width 0.25) (layer F.Cu) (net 10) (status 400000))
 (segment (start 135.89 105.41) (end 139.541 105.41) (width 0.25) (layer F.Cu) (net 10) (status 800000))
 (segment (start 133.35 102.87) (end 135.89 105.41) (width 0.25) (layer F.Cu) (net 10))
 (segment (start 139.541 107.95) (end 135.89 107.95) (width 0.25) (layer F.Cu) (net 11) (status 400000))
 (segment (start 133.35 105.41) (end 129.54 105.41) (width 0.25) (layer F.Cu) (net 11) (status 800000))
 (segment (start 135.89 107.95) (end 133.35 105.41) (width 0.25) (layer F.Cu) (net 11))
 (segment (start 129.54 107.95) (end 133.35 107.95) (width 0.25) (layer F.Cu) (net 12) (status 400000))
 (segment (start 135.89 110.49) (end 139.541 110.49) (width 0.25) (layer F.Cu) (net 12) (status 800000))
 (segment (start 133.35 107.95) (end 135.89 110.49) (width 0.25) (layer F.Cu) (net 12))
 (segment (start 139.541 115.57) (end 139.541 122.079) (width 0.25) (layer F.Cu) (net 14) (status 400000))
 (segment (start 138.43 123.19) (end 138.43 129.54) (width 0.25) (layer F.Cu) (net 14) (status 800000))
 (segment (start 139.541 122.079) (end 138.43 123.19) (width 0.25) (layer F.Cu) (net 14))
 (segment (start 147.479 115.57) (end 147.479 116.681) (width 0.25) (layer F.Cu) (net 15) (status 400000))
 (segment (start 140.97 123.19) (end 140.97 129.54) (width 0.25) (layer F.Cu) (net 15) (status 800000))
 (segment (start 147.479 116.681) (end 140.97 123.19) (width 0.25) (layer F.Cu) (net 15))
 (segment (start 129.54 116.84) (end 129.54 116.84) (width 0.25) (layer B.Cu) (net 16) (status C00000))
 (segment (start 138.589 121.92) (end 147.479 113.03) (width 0.25) (layer B.Cu) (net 16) (status 800000))
 (segment (start 134.62 121.92) (end 138.589 121.92) (width 0.25) (layer B.Cu) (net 16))
 (segment (start 129.54 116.84) (end 134.62 121.92) (width 0.25) (layer B.Cu) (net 16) (status 400000))
 (segment (start 156.21 95.25) (end 153.67 97.79) (width 0.25) (layer B.Cu) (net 17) (status 400000))
 (segment (start 151.13 110.49) (end 147.479 110.49) (width 0.25) (layer B.Cu) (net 17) (status 800000))
 (segment (start 153.67 107.95) (end 151.13 110.49) (width 0.25) (layer B.Cu) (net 17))
 (segment (start 153.67 97.79) (end 153.67 107.95) (width 0.25) (layer B.Cu) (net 17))
 (segment (start 147.479 107.95) (end 147.479 107.791) (width 0.25) (layer F.Cu) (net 18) (status C00000))
 (segment (start 153.67 92.71) (end 156.21 92.71) (width 0.25) (layer F.Cu) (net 18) (status 800000))
 (segment (start 152.4 93.98) (end 153.67 92.71) (width 0.25) (layer F.Cu) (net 18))
 (segment (start 152.4 97.79) (end 152.4 93.98) (width 0.25) (layer F.Cu) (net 18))
 (segment (start 148.59 101.6) (end 152.4 97.79) (width 0.25) (layer F.Cu) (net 18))
 (segment (start 148.59 106.68) (end 148.59 101.6) (width 0.25) (layer F.Cu) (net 18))
 (segment (start 147.479 107.791) (end 148.59 106.68) (width 0.25) (layer F.Cu) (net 18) (status 400000))
 (segment (start 156.21 90.17) (end 153.67 90.17) (width 0.25) (layer F.Cu) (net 20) (status 400000))
 (segment (start 151.13 96.679) (end 147.479 100.33) (width 0.25) (layer F.Cu) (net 20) (status 800000))
 (segment (start 151.13 92.71) (end 151.13 96.679) (width 0.25) (layer F.Cu) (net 20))
 (segment (start 153.67 90.17) (end 151.13 92.71) (width 0.25) (layer F.Cu) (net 20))
 (segment (start 156.21 87.63) (end 153.67 87.63) (width 0.25) (layer F.Cu) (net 21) (status 400000))
 (segment (start 149.86 95.409) (end 147.479 97.79) (width 0.25) (layer F.Cu) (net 21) (status 800000))
 (segment (start 149.86 91.44) (end 149.86 95.409) (width 0.25) (layer F.Cu) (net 21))
 (segment (start 153.67 87.63) (end 149.86 91.44) (width 0.25) (layer F.Cu) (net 21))
 (segment (start 147.479 95.25) (end 146.05 95.25) (width 0.25) (layer B.Cu) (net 22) (status 400000))
 (segment (start 152.4 113.03) (end 156.21 113.03) (width 0.25) (layer B.Cu) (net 22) (status 800000))
 (segment (start 151.13 111.76) (end 152.4 113.03) (width 0.25) (layer B.Cu) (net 22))
 (segment (start 146.05 111.76) (end 151.13 111.76) (width 0.25) (layer B.Cu) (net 22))
 (segment (start 144.78 110.49) (end 146.05 111.76) (width 0.25) (layer B.Cu) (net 22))
 (segment (start 144.78 96.52) (end 144.78 110.49) (width 0.25) (layer B.Cu) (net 22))
 (segment (start 146.05 95.25) (end 144.78 96.52) (width 0.25) (layer B.Cu) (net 22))
 (segment (start 156.21 107.95) (end 158.75 105.41) (width 0.25) (layer B.Cu) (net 23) (status 400000))
 (segment (start 153.67 86.519) (end 147.479 92.71) (width 0.25) (layer B.Cu) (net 23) (status 800000))
 (segment (start 153.67 81.28) (end 153.67 86.519) (width 0.25) (layer B.Cu) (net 23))
 (segment (start 154.94 80.01) (end 153.67 81.28) (width 0.25) (layer B.Cu) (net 23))
 (segment (start 157.48 80.01) (end 154.94 80.01) (width 0.25) (layer B.Cu) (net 23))
 (segment (start 158.75 81.28) (end 157.48 80.01) (width 0.25) (layer B.Cu) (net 23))
 (segment (start 158.75 82.55) (end 158.75 81.28) (width 0.25) (layer B.Cu) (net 23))
 (segment (start 158.75 105.41) (end 158.75 82.55) (width 0.25) (layer B.Cu) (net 23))
 (segment (start 147.479 90.17) (end 147.32 90.17) (width 0.25) (layer B.Cu) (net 24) (status C00000))
 (segment (start 134.62 119.38) (end 129.54 114.3) (width 0.25) (layer B.Cu) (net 24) (status 800000))
 (segment (start 138.43 119.38) (end 134.62 119.38) (width 0.25) (layer B.Cu) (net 24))
 (segment (start 143.51 114.3) (end 138.43 119.38) (width 0.25) (layer B.Cu) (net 24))
 (segment (start 143.51 93.98) (end 143.51 114.3) (width 0.25) (layer B.Cu) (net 24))
 (segment (start 147.32 90.17) (end 143.51 93.98) (width 0.25) (layer B.Cu) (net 24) (status 400000))
 (segment (start 147.479 87.63) (end 144.78 87.63) (width 0.25) (layer B.Cu) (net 25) (status 400000))
 (segment (start 132.08 111.76) (end 129.54 111.76) (width 0.25) (layer B.Cu) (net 25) (status 800000))
 (segment (start 133.35 110.49) (end 132.08 111.76) (width 0.25) (layer B.Cu) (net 25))
 (segment (start 135.89 110.49) (end 133.35 110.49) (width 0.25) (layer B.Cu) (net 25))
 (segment (start 137.16 111.76) (end 135.89 110.49) (width 0.25) (layer B.Cu) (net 25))
 (segment (start 137.16 113.03) (end 137.16 111.76) (width 0.25) (layer B.Cu) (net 25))
 (segment (start 138.43 114.3) (end 137.16 113.03) (width 0.25) (layer B.Cu) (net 25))
 (segment (start 140.97 114.3) (end 138.43 114.3) (width 0.25) (layer B.Cu) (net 25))
 (segment (start 142.24 113.03) (end 140.97 114.3) (width 0.25) (layer B.Cu) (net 25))
 (segment (start 142.24 90.17) (end 142.24 113.03) (width 0.25) (layer B.Cu) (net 25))
 (segment (start 144.78 87.63) (end 142.24 90.17) (width 0.25) (layer B.Cu) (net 25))
 (segment (start 148.59 120.69) (end 148.59 118.11) (width 0.25) (layer F.Cu) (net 27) (status 400000))
 (segment (start 151.13 115.57) (end 156.21 115.57) (width 0.25) (layer F.Cu) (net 27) (status 800000))
 (segment (start 148.59 118.11) (end 151.13 115.57) (width 0.25) (layer F.Cu) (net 27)))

